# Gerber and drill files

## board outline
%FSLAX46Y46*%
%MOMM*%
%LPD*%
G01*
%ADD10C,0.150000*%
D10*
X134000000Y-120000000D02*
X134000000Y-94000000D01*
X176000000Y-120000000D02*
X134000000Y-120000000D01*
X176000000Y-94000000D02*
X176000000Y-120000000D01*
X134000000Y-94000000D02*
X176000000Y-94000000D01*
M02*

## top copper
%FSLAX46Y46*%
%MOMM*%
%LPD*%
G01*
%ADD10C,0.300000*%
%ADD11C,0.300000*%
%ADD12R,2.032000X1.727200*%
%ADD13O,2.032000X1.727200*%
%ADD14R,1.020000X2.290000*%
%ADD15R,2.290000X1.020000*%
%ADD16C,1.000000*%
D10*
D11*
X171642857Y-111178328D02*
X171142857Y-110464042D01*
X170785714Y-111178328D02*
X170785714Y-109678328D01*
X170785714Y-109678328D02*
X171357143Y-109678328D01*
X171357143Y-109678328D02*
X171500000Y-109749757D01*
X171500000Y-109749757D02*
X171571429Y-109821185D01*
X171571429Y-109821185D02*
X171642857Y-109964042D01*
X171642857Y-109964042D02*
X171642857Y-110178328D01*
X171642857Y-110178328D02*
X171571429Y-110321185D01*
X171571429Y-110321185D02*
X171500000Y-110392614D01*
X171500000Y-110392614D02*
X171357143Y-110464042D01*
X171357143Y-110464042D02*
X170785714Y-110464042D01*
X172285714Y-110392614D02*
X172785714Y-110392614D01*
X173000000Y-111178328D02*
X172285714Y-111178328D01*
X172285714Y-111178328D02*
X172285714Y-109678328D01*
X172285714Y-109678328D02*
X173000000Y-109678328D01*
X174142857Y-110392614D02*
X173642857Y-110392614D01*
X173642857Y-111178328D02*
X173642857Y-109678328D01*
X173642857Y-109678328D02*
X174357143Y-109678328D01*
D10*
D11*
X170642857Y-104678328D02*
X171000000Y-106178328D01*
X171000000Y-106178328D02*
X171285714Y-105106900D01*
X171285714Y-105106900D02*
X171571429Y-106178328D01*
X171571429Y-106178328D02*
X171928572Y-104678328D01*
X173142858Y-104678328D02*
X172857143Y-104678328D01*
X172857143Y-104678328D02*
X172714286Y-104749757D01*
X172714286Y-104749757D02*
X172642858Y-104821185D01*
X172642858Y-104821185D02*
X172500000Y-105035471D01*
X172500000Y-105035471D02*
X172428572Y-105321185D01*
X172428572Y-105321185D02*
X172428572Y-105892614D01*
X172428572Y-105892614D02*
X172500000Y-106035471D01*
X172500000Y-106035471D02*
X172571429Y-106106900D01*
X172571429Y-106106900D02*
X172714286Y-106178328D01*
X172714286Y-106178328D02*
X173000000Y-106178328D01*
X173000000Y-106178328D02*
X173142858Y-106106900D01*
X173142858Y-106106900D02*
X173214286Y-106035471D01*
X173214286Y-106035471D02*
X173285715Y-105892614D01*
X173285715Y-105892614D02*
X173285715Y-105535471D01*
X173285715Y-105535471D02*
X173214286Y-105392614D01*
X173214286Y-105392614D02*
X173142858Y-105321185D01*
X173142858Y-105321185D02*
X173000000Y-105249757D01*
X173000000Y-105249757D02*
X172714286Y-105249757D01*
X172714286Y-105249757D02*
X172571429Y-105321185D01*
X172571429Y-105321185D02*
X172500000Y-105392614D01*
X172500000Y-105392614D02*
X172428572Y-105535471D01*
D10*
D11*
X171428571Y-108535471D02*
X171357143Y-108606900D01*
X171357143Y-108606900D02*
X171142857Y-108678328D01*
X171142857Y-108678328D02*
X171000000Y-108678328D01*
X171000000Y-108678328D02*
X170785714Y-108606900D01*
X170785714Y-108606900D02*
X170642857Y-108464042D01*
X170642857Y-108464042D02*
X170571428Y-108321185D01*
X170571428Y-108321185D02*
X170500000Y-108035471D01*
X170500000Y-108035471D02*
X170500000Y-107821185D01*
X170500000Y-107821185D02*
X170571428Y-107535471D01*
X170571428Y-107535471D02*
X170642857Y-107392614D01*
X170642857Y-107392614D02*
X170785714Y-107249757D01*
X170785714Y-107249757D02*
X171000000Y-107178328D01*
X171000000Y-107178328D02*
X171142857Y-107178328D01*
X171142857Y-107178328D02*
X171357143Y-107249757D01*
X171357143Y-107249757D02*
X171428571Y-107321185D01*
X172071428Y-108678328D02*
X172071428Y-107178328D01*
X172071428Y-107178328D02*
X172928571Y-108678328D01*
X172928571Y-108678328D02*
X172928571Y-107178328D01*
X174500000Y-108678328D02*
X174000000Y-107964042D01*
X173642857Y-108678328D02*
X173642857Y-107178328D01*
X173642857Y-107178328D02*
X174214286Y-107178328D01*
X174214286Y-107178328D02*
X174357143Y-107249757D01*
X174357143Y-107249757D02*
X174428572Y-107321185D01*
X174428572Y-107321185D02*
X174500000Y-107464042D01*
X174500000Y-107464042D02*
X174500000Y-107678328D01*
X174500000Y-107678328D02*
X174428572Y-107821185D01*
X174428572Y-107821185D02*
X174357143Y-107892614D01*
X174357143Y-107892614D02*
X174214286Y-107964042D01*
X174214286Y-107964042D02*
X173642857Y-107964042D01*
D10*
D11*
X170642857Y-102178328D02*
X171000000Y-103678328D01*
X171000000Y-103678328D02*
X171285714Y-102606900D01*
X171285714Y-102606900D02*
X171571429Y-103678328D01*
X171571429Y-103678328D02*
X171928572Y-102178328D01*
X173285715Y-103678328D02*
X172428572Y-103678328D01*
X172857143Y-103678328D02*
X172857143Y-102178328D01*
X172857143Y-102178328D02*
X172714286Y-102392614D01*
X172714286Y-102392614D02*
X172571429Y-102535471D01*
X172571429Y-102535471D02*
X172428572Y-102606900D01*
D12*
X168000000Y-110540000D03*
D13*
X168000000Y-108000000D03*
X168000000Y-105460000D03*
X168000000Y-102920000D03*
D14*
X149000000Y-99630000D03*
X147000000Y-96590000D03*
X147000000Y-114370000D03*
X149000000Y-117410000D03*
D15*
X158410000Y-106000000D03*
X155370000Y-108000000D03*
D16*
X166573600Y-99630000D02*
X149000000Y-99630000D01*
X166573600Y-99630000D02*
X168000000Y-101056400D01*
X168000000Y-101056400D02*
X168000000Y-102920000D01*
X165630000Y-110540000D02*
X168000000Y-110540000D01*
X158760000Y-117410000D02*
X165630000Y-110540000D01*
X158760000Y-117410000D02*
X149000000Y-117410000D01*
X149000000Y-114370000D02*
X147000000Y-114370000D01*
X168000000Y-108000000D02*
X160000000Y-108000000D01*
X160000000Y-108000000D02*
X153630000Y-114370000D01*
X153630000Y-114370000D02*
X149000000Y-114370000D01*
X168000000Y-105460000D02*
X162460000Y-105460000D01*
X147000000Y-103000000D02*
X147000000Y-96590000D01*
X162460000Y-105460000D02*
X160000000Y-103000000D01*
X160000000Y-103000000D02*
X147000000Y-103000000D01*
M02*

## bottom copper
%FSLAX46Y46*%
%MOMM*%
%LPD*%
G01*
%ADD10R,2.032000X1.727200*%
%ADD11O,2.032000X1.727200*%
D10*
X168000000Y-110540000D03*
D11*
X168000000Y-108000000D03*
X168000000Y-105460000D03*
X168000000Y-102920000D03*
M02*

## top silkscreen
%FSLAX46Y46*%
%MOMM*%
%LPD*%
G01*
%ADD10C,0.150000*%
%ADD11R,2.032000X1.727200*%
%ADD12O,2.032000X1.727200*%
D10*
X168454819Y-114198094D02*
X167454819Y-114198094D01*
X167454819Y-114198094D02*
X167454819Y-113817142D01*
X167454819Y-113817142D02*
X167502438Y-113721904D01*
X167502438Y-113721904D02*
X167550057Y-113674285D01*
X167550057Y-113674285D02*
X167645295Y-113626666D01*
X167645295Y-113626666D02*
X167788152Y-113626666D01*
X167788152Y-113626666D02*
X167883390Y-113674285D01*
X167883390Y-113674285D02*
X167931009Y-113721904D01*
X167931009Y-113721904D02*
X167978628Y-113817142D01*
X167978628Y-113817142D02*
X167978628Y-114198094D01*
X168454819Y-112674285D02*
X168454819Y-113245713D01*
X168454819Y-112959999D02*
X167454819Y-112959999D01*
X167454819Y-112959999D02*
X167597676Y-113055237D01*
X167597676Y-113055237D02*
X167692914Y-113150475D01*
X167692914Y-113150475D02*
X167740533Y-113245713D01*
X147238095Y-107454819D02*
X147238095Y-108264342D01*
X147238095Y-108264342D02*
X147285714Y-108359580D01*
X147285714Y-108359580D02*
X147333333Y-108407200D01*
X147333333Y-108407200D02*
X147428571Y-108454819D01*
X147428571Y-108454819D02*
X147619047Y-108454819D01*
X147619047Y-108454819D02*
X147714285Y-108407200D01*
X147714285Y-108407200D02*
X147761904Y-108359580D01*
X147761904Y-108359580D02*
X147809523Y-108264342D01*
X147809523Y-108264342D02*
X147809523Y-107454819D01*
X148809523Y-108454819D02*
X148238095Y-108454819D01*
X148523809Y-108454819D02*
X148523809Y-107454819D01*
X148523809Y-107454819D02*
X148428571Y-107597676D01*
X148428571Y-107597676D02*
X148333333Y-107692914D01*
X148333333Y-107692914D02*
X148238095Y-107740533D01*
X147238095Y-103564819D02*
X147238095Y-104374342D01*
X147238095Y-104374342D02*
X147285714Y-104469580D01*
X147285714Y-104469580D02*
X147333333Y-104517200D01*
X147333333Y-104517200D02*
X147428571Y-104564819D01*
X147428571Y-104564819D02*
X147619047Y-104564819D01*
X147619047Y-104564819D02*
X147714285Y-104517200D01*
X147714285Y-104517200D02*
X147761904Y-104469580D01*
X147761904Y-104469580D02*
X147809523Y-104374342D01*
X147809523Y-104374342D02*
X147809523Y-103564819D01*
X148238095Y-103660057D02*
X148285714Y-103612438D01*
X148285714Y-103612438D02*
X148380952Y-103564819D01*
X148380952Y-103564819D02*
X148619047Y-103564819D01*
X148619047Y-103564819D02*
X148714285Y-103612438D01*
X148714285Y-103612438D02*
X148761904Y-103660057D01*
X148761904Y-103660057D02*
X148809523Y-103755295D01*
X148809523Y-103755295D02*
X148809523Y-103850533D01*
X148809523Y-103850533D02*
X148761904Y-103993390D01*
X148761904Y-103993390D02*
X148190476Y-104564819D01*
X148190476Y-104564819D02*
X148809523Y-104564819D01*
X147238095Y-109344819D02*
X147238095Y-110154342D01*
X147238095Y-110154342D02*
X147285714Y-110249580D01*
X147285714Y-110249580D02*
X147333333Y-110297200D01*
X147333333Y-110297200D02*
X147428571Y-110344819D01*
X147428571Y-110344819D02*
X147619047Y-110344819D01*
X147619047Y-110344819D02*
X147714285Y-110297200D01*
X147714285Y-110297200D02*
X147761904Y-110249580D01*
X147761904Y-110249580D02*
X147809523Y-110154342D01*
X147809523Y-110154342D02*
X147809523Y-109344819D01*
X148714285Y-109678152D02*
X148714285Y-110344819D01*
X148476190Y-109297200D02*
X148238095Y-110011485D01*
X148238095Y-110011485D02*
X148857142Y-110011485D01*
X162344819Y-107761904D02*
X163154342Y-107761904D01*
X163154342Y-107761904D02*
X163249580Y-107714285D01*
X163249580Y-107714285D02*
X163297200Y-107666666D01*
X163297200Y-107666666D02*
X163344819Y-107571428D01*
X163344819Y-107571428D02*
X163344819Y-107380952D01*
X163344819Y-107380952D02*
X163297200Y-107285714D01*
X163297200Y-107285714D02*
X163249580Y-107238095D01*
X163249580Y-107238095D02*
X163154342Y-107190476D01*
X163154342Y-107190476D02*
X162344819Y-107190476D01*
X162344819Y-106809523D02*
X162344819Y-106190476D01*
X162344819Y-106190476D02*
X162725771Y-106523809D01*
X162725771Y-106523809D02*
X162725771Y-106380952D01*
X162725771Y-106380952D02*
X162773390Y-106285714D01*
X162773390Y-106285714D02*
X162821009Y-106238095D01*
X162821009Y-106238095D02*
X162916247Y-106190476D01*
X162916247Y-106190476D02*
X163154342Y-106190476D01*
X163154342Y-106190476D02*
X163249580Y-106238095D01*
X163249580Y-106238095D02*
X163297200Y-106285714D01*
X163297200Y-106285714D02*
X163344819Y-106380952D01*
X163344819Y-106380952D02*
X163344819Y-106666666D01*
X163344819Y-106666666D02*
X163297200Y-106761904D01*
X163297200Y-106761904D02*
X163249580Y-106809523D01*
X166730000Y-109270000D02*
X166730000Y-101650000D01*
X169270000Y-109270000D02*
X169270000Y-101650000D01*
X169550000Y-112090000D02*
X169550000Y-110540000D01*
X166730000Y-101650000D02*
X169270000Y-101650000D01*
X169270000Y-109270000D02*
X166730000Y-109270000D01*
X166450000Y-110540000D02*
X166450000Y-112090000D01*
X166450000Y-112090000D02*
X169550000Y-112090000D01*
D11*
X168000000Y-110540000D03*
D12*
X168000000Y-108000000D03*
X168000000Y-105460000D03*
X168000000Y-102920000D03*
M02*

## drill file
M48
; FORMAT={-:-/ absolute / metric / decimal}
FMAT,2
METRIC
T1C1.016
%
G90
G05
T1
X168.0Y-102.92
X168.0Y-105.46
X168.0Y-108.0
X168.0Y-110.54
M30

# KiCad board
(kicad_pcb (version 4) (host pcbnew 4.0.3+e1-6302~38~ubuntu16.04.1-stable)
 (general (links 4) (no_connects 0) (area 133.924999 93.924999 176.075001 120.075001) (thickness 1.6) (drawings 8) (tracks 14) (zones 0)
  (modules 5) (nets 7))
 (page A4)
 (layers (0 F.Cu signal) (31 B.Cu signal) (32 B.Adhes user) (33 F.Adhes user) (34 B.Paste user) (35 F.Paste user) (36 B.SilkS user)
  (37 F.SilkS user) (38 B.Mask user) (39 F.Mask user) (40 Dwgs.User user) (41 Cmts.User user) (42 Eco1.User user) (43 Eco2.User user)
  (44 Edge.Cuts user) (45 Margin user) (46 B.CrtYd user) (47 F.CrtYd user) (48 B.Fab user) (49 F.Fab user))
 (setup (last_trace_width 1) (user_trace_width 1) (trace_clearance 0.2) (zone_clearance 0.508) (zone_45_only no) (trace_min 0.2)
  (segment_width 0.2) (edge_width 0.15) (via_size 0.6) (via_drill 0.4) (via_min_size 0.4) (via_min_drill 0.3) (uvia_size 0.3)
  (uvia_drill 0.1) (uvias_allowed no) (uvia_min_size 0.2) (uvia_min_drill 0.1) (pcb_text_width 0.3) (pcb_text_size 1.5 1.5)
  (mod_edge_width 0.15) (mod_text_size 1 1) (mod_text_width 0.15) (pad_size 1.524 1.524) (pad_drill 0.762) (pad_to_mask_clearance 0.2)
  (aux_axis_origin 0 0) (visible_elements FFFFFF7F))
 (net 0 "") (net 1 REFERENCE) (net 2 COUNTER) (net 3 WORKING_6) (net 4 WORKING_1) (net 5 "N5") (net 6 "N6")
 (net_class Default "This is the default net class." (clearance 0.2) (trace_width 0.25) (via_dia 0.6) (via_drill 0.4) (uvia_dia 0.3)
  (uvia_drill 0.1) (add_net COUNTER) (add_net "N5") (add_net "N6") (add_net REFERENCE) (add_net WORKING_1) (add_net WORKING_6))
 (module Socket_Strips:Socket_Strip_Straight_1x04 (layer F.Cu) (at 168 110.54 90)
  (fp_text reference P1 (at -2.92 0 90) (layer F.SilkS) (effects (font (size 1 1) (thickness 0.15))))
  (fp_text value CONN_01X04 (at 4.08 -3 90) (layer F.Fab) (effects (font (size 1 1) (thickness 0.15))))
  (fp_line (start 1.27 -1.27) (end 8.89 -1.27) (layer F.SilkS) (width 0.15))
  (fp_line (start 1.27 1.27) (end 8.89 1.27) (layer F.SilkS) (width 0.15))
  (fp_line (start -1.55 1.55) (end 0 1.55) (layer F.SilkS) (width 0.15))
  (fp_line (start 8.89 -1.27) (end 8.89 1.27) (layer F.SilkS) (width 0.15))
  (fp_line (start 1.27 1.27) (end 1.27 -1.27) (layer F.SilkS) (width 0.15))
  (fp_line (start 0 -1.55) (end -1.55 -1.55) (layer F.SilkS) (width 0.15))
  (fp_line (start -1.55 -1.55) (end -1.55 1.55) (layer F.SilkS) (width 0.15))
  (pad 1 thru_hole rect (at 0 0 90) (size 1.7272 2.032) (drill 1.016) (layers *.Cu *.Mask F.SilkS) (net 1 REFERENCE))
  (pad 2 thru_hole oval (at 2.54 0 90) (size 1.7272 2.032) (drill 1.016) (layers *.Cu *.Mask F.SilkS) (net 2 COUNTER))
  (pad 3 thru_hole oval (at 5.08 0 90) (size 1.7272 2.032) (drill 1.016) (layers *.Cu *.Mask F.SilkS) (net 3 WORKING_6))
  (pad 4 thru_hole oval (at 7.62 0 90) (size 1.7272 2.032) (drill 1.016) (layers *.Cu *.Mask F.SilkS) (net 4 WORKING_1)))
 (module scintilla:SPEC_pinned (layer F.Cu) (at 148 107)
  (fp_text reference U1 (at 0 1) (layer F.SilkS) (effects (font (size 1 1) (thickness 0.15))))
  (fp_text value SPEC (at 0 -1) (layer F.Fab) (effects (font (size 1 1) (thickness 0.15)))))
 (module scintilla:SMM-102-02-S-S (layer F.Cu) (at 148 98.11)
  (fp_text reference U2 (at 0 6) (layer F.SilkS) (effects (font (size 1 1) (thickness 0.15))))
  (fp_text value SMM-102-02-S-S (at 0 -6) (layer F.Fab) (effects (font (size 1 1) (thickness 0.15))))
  (pad 1 smd rect (at 1 1.52) (size 1.02 2.29) (layers F.Cu F.Paste F.Mask) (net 4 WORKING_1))
  (pad 2 smd rect (at -1 -1.52) (size 1.02 2.29) (layers F.Cu F.Paste F.Mask) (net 3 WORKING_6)))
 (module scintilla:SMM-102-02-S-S (layer F.Cu) (at 148 115.89 180)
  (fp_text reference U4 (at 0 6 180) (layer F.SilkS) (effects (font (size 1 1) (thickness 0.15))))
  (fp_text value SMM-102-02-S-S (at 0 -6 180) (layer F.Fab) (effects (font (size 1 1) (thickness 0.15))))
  (pad 1 smd rect (at 1 1.52 180) (size 1.02 2.29) (layers F.Cu F.Paste F.Mask) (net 2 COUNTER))
  (pad 2 smd rect (at -1 -1.52 180) (size 1.02 2.29) (layers F.Cu F.Paste F.Mask) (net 1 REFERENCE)))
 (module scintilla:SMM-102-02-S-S (layer F.Cu) (at 156.89 107 90)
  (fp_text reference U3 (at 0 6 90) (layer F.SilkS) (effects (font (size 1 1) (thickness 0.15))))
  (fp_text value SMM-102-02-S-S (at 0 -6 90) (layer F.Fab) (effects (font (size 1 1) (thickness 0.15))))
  (pad 1 smd rect (at 1 1.52 90) (size 1.02 2.29) (layers F.Cu F.Paste F.Mask) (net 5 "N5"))
  (pad 2 smd rect (at -1 -1.52 90) (size 1.02 2.29) (layers F.Cu F.Paste F.Mask) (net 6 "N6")))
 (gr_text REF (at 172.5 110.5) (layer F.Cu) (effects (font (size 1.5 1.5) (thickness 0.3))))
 (gr_line (start 134 120) (end 134 94) (layer Edge.Cuts) (width 0.15))
 (gr_line (start 176 120) (end 134 120) (layer Edge.Cuts) (width 0.15))
 (gr_line (start 176 94) (end 176 120) (layer Edge.Cuts) (width 0.15))
 (gr_line (start 134 94) (end 176 94) (layer Edge.Cuts) (width 0.15))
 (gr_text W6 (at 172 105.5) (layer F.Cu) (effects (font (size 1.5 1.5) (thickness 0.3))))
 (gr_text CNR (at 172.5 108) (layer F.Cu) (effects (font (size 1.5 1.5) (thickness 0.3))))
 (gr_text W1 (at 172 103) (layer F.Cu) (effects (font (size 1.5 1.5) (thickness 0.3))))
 (segment (start 166.5736 99.63) (end 149 99.63) (width 1) (layer F.Cu) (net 4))
 (segment (start 166.5736 99.63) (end 168 101.0564) (width 1) (layer F.Cu) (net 4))
 (segment (start 168 101.0564) (end 168 102.92) (width 1) (layer F.Cu) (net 4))
 (segment (start 165.63 110.54) (end 168 110.54) (width 1) (layer F.Cu) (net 1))
 (segment (start 158.76 117.41) (end 165.63 110.54) (width 1) (layer F.Cu) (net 1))
 (segment (start 158.76 117.41) (end 149 117.41) (width 1) (layer F.Cu) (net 1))
 (segment (start 149 114.37) (end 147 114.37) (width 1) (layer F.Cu) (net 2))
 (segment (start 168 108) (end 160 108) (width 1) (layer F.Cu) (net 2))
 (segment (start 160 108) (end 153.63 114.37) (width 1) (layer F.Cu) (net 2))
 (segment (start 153.63 114.37) (end 149 114.37) (width 1) (layer F.Cu) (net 2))
 (segment (start 168 105.46) (end 162.46 105.46) (width 1) (layer F.Cu) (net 3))
 (segment (start 147 103) (end 147 96.59) (width 1) (layer F.Cu) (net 3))
 (segment (start 162.46 105.46) (end 160 103) (width 1) (layer F.Cu) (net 3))
 (segment (start 160 103) (end 147 103) (width 1) (layer F.Cu) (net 3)))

